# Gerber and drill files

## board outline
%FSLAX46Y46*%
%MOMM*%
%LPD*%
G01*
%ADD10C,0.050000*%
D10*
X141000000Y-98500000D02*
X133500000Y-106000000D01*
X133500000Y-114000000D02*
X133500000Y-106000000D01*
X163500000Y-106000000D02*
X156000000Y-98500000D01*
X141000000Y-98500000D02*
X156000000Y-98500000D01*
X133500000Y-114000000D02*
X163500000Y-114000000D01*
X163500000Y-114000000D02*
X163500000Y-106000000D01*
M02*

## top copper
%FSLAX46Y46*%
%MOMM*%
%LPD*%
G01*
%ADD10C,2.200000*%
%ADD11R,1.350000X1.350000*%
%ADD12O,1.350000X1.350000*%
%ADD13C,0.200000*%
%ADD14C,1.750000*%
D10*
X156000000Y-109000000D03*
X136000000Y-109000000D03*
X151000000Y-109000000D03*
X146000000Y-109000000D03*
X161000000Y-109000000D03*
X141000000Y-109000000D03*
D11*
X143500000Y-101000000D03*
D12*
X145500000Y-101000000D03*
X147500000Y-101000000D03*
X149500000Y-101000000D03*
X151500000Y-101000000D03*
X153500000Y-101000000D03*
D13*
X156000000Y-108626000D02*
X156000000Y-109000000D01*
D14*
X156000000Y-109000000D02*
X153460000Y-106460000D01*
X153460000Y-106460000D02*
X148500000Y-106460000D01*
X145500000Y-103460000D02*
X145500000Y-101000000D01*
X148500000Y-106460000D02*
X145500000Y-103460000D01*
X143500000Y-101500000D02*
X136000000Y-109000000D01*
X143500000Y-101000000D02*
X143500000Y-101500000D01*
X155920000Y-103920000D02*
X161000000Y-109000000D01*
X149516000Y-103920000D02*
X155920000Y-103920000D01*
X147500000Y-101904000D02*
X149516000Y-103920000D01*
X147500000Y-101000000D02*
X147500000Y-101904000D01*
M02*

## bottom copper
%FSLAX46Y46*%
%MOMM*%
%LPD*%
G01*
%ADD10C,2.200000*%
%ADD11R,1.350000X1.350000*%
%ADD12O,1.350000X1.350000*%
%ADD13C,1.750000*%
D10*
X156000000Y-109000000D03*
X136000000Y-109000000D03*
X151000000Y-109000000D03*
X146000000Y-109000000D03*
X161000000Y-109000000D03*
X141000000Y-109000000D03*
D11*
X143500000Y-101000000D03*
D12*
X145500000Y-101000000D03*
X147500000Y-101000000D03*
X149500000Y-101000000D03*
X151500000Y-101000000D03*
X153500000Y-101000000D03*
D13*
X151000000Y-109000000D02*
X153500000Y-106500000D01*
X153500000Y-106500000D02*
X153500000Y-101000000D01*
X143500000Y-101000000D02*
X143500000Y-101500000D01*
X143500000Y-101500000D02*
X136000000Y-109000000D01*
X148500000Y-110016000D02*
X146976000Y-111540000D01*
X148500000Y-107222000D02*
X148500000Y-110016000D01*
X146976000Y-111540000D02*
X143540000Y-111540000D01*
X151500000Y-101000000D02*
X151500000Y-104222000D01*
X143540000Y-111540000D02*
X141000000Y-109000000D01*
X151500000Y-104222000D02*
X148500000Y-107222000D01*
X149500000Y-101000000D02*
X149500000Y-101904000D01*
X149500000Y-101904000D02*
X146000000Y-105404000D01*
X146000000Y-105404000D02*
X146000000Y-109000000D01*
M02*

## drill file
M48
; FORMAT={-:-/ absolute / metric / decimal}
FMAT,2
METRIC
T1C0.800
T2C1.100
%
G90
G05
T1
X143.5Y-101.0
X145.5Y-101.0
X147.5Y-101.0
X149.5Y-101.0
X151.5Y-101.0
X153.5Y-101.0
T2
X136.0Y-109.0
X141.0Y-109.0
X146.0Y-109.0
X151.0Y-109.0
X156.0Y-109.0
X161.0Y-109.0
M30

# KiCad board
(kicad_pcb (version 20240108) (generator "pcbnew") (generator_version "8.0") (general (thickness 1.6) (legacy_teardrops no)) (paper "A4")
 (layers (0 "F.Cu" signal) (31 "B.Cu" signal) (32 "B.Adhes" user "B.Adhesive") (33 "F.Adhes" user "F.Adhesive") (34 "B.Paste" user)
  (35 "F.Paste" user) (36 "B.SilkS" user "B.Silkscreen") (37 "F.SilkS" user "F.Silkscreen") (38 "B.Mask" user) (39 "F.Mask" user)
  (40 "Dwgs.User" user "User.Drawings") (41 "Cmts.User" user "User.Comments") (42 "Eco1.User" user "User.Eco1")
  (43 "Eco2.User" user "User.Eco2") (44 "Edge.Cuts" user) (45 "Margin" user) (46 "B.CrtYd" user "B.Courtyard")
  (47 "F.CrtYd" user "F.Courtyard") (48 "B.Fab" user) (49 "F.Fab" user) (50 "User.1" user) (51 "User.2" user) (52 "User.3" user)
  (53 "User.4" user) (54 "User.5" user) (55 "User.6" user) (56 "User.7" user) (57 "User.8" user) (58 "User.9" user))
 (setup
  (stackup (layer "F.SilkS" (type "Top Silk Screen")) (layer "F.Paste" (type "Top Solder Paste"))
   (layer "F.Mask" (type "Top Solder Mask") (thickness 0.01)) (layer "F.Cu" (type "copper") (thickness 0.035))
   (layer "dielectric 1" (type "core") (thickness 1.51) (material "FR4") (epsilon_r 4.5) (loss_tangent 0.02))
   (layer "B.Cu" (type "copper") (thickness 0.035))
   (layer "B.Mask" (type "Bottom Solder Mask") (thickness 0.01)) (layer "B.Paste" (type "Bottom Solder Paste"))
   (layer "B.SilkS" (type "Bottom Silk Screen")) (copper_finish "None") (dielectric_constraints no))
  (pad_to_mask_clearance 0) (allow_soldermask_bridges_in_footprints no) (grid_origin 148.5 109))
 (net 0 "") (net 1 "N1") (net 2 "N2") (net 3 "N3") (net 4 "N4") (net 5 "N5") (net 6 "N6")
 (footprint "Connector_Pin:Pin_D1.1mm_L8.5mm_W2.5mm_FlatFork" (layer "F.Cu") (at 156 109 90)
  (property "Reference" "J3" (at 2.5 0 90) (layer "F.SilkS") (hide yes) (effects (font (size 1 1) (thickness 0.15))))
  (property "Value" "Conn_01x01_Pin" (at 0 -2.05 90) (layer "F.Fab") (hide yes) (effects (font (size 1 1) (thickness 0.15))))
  (pad "1" thru_hole circle (at 0 0 90) (size 2.2 2.2) (drill 1.1) (layers "*.Cu" "*.Mask") (remove_unused_layers no) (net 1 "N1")))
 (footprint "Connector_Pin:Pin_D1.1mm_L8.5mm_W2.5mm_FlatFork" (layer "F.Cu") (at 136 109 90)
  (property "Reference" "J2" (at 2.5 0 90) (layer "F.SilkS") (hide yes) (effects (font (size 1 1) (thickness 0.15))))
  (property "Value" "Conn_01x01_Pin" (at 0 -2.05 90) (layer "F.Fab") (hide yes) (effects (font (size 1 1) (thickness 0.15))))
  (pad "1" thru_hole circle (at 0 0 90) (size 2.2 2.2) (drill 1.1) (layers "*.Cu" "*.Mask") (remove_unused_layers no) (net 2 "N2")))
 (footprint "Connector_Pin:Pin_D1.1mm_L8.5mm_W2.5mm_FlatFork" (layer "F.Cu") (at 151 109 90)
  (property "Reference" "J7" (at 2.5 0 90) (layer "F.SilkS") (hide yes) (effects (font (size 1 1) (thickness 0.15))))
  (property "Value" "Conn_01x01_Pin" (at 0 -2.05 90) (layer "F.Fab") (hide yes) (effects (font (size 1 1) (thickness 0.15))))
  (pad "1" thru_hole circle (at 0 0 90) (size 2.2 2.2) (drill 1.1) (layers "*.Cu" "*.Mask") (remove_unused_layers no) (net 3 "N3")))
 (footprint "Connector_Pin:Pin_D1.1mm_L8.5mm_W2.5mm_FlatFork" (layer "F.Cu") (at 146 109 90)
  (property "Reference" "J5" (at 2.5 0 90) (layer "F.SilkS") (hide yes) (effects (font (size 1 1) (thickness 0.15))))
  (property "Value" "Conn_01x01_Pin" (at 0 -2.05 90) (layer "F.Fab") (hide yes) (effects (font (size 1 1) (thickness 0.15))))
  (pad "1" thru_hole circle (at 0 0 90) (size 2.2 2.2) (drill 1.1) (layers "*.Cu" "*.Mask") (remove_unused_layers no) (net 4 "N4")))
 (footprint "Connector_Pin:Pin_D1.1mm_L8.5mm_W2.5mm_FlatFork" (layer "F.Cu") (at 161 109 90)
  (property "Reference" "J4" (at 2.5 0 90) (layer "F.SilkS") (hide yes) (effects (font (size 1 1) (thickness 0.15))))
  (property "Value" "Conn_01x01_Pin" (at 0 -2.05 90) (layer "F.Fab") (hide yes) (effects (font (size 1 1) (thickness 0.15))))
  (pad "1" thru_hole circle (at 0 0 90) (size 2.2 2.2) (drill 1.1) (layers "*.Cu" "*.Mask") (remove_unused_layers no) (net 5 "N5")))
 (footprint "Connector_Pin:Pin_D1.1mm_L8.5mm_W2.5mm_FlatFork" (layer "F.Cu") (at 141 109 90)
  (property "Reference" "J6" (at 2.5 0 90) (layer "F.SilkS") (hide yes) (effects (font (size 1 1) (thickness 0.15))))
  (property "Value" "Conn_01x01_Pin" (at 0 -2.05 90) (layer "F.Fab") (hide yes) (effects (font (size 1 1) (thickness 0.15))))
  (pad "1" thru_hole circle (at 0 0 90) (size 2.2 2.2) (drill 1.1) (layers "*.Cu" "*.Mask") (remove_unused_layers no) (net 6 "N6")))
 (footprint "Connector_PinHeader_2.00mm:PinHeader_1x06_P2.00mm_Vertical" (layer "B.Cu") (at 143.5 101 -90)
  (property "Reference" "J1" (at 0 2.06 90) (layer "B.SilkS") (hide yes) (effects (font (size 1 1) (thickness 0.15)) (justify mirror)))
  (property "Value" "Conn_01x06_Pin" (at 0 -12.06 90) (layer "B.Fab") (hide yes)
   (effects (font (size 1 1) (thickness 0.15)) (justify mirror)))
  (pad "1" thru_hole rect (at 0 0 270) (size 1.35 1.35) (drill 0.8) (layers "*.Cu" "*.Mask") (remove_unused_layers no) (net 2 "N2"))
  (pad "2" thru_hole oval (at 0 -2 270) (size 1.35 1.35) (drill 0.8) (layers "*.Cu" "*.Mask") (remove_unused_layers no) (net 1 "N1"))
  (pad "3" thru_hole oval (at 0 -4 270) (size 1.35 1.35) (drill 0.8) (layers "*.Cu" "*.Mask") (remove_unused_layers no) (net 5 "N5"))
  (pad "4" thru_hole oval (at 0 -6 270) (size 1.35 1.35) (drill 0.8) (layers "*.Cu" "*.Mask") (remove_unused_layers no) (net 4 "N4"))
  (pad "5" thru_hole oval (at 0 -8 270) (size 1.35 1.35) (drill 0.8) (layers "*.Cu" "*.Mask") (remove_unused_layers no) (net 6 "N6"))
  (pad "6" thru_hole oval (at 0 -10 270) (size 1.35 1.35) (drill 0.8) (layers "*.Cu" "*.Mask") (remove_unused_layers no) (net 3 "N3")))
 (gr_line (start 141 98.5) (end 133.5 106) (stroke (width 0.05) (type default)) (layer "Edge.Cuts"))
 (gr_line (start 133.5 114) (end 133.5 106) (stroke (width 0.05) (type default)) (layer "Edge.Cuts"))
 (gr_line (start 163.5 106) (end 156 98.5) (stroke (width 0.05) (type default)) (layer "Edge.Cuts"))
 (gr_line (start 141 98.5) (end 156 98.5) (stroke (width 0.05) (type default)) (layer "Edge.Cuts"))
 (gr_line (start 133.5 114) (end 163.5 114) (stroke (width 0.05) (type default)) (layer "Edge.Cuts"))
 (gr_line (start 163.5 114) (end 163.5 106) (stroke (width 0.05) (type default)) (layer "Edge.Cuts"))
 (segment (start 151 109) (end 153.5 106.5) (width 1.75) (layer "B.Cu") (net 3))
 (segment (start 153.5 106.5) (end 153.5 101) (width 1.75) (layer "B.Cu") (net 3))
 (segment (start 156 108.626) (end 156 109) (width 0.2) (layer "F.Cu") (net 1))
 (segment (start 156 109) (end 153.46 106.46) (width 1.75) (layer "F.Cu") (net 1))
 (segment (start 153.46 106.46) (end 148.5 106.46) (width 1.75) (layer "F.Cu") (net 1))
 (segment (start 145.5 103.46) (end 145.5 101) (width 1.75) (layer "F.Cu") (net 1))
 (segment (start 148.5 106.46) (end 145.5 103.46) (width 1.75) (layer "F.Cu") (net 1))
 (segment (start 143.5 101.5) (end 136 109) (width 1.75) (layer "F.Cu") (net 2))
 (segment (start 143.5 101) (end 143.5 101.5) (width 1.75) (layer "F.Cu") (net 2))
 (segment (start 143.5 101) (end 143.5 101.5) (width 1.75) (layer "B.Cu") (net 2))
 (segment (start 143.5 101.5) (end 136 109) (width 1.75) (layer "B.Cu") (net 2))
 (segment (start 148.5 110.016) (end 146.976 111.54) (width 1.75) (layer "B.Cu") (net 6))
 (segment (start 148.5 107.222) (end 148.5 110.016) (width 1.75) (layer "B.Cu") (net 6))
 (segment (start 146.976 111.54) (end 143.54 111.54) (width 1.75) (layer "B.Cu") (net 6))
 (segment (start 151.5 101) (end 151.5 104.222) (width 1.75) (layer "B.Cu") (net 6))
 (segment (start 143.54 111.54) (end 141 109) (width 1.75) (layer "B.Cu") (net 6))
 (segment (start 151.5 104.222) (end 148.5 107.222) (width 1.75) (layer "B.Cu") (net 6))
 (segment (start 149.5 101) (end 149.5 101.904) (width 1.75) (layer "B.Cu") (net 4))
 (segment (start 149.5 101.904) (end 146 105.404) (width 1.75) (layer "B.Cu") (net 4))
 (segment (start 146 105.404) (end 146 109) (width 1.75) (layer "B.Cu") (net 4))
 (segment (start 155.92 103.92) (end 161 109) (width 1.75) (layer "F.Cu") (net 5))
 (segment (start 149.516 103.92) (end 155.92 103.92) (width 1.75) (layer "F.Cu") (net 5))
 (segment (start 147.5 101.904) (end 149.516 103.92) (width 1.75) (layer "F.Cu") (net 5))
 (segment (start 147.5 101) (end 147.5 101.904) (width 1.75) (layer "F.Cu") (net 5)))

